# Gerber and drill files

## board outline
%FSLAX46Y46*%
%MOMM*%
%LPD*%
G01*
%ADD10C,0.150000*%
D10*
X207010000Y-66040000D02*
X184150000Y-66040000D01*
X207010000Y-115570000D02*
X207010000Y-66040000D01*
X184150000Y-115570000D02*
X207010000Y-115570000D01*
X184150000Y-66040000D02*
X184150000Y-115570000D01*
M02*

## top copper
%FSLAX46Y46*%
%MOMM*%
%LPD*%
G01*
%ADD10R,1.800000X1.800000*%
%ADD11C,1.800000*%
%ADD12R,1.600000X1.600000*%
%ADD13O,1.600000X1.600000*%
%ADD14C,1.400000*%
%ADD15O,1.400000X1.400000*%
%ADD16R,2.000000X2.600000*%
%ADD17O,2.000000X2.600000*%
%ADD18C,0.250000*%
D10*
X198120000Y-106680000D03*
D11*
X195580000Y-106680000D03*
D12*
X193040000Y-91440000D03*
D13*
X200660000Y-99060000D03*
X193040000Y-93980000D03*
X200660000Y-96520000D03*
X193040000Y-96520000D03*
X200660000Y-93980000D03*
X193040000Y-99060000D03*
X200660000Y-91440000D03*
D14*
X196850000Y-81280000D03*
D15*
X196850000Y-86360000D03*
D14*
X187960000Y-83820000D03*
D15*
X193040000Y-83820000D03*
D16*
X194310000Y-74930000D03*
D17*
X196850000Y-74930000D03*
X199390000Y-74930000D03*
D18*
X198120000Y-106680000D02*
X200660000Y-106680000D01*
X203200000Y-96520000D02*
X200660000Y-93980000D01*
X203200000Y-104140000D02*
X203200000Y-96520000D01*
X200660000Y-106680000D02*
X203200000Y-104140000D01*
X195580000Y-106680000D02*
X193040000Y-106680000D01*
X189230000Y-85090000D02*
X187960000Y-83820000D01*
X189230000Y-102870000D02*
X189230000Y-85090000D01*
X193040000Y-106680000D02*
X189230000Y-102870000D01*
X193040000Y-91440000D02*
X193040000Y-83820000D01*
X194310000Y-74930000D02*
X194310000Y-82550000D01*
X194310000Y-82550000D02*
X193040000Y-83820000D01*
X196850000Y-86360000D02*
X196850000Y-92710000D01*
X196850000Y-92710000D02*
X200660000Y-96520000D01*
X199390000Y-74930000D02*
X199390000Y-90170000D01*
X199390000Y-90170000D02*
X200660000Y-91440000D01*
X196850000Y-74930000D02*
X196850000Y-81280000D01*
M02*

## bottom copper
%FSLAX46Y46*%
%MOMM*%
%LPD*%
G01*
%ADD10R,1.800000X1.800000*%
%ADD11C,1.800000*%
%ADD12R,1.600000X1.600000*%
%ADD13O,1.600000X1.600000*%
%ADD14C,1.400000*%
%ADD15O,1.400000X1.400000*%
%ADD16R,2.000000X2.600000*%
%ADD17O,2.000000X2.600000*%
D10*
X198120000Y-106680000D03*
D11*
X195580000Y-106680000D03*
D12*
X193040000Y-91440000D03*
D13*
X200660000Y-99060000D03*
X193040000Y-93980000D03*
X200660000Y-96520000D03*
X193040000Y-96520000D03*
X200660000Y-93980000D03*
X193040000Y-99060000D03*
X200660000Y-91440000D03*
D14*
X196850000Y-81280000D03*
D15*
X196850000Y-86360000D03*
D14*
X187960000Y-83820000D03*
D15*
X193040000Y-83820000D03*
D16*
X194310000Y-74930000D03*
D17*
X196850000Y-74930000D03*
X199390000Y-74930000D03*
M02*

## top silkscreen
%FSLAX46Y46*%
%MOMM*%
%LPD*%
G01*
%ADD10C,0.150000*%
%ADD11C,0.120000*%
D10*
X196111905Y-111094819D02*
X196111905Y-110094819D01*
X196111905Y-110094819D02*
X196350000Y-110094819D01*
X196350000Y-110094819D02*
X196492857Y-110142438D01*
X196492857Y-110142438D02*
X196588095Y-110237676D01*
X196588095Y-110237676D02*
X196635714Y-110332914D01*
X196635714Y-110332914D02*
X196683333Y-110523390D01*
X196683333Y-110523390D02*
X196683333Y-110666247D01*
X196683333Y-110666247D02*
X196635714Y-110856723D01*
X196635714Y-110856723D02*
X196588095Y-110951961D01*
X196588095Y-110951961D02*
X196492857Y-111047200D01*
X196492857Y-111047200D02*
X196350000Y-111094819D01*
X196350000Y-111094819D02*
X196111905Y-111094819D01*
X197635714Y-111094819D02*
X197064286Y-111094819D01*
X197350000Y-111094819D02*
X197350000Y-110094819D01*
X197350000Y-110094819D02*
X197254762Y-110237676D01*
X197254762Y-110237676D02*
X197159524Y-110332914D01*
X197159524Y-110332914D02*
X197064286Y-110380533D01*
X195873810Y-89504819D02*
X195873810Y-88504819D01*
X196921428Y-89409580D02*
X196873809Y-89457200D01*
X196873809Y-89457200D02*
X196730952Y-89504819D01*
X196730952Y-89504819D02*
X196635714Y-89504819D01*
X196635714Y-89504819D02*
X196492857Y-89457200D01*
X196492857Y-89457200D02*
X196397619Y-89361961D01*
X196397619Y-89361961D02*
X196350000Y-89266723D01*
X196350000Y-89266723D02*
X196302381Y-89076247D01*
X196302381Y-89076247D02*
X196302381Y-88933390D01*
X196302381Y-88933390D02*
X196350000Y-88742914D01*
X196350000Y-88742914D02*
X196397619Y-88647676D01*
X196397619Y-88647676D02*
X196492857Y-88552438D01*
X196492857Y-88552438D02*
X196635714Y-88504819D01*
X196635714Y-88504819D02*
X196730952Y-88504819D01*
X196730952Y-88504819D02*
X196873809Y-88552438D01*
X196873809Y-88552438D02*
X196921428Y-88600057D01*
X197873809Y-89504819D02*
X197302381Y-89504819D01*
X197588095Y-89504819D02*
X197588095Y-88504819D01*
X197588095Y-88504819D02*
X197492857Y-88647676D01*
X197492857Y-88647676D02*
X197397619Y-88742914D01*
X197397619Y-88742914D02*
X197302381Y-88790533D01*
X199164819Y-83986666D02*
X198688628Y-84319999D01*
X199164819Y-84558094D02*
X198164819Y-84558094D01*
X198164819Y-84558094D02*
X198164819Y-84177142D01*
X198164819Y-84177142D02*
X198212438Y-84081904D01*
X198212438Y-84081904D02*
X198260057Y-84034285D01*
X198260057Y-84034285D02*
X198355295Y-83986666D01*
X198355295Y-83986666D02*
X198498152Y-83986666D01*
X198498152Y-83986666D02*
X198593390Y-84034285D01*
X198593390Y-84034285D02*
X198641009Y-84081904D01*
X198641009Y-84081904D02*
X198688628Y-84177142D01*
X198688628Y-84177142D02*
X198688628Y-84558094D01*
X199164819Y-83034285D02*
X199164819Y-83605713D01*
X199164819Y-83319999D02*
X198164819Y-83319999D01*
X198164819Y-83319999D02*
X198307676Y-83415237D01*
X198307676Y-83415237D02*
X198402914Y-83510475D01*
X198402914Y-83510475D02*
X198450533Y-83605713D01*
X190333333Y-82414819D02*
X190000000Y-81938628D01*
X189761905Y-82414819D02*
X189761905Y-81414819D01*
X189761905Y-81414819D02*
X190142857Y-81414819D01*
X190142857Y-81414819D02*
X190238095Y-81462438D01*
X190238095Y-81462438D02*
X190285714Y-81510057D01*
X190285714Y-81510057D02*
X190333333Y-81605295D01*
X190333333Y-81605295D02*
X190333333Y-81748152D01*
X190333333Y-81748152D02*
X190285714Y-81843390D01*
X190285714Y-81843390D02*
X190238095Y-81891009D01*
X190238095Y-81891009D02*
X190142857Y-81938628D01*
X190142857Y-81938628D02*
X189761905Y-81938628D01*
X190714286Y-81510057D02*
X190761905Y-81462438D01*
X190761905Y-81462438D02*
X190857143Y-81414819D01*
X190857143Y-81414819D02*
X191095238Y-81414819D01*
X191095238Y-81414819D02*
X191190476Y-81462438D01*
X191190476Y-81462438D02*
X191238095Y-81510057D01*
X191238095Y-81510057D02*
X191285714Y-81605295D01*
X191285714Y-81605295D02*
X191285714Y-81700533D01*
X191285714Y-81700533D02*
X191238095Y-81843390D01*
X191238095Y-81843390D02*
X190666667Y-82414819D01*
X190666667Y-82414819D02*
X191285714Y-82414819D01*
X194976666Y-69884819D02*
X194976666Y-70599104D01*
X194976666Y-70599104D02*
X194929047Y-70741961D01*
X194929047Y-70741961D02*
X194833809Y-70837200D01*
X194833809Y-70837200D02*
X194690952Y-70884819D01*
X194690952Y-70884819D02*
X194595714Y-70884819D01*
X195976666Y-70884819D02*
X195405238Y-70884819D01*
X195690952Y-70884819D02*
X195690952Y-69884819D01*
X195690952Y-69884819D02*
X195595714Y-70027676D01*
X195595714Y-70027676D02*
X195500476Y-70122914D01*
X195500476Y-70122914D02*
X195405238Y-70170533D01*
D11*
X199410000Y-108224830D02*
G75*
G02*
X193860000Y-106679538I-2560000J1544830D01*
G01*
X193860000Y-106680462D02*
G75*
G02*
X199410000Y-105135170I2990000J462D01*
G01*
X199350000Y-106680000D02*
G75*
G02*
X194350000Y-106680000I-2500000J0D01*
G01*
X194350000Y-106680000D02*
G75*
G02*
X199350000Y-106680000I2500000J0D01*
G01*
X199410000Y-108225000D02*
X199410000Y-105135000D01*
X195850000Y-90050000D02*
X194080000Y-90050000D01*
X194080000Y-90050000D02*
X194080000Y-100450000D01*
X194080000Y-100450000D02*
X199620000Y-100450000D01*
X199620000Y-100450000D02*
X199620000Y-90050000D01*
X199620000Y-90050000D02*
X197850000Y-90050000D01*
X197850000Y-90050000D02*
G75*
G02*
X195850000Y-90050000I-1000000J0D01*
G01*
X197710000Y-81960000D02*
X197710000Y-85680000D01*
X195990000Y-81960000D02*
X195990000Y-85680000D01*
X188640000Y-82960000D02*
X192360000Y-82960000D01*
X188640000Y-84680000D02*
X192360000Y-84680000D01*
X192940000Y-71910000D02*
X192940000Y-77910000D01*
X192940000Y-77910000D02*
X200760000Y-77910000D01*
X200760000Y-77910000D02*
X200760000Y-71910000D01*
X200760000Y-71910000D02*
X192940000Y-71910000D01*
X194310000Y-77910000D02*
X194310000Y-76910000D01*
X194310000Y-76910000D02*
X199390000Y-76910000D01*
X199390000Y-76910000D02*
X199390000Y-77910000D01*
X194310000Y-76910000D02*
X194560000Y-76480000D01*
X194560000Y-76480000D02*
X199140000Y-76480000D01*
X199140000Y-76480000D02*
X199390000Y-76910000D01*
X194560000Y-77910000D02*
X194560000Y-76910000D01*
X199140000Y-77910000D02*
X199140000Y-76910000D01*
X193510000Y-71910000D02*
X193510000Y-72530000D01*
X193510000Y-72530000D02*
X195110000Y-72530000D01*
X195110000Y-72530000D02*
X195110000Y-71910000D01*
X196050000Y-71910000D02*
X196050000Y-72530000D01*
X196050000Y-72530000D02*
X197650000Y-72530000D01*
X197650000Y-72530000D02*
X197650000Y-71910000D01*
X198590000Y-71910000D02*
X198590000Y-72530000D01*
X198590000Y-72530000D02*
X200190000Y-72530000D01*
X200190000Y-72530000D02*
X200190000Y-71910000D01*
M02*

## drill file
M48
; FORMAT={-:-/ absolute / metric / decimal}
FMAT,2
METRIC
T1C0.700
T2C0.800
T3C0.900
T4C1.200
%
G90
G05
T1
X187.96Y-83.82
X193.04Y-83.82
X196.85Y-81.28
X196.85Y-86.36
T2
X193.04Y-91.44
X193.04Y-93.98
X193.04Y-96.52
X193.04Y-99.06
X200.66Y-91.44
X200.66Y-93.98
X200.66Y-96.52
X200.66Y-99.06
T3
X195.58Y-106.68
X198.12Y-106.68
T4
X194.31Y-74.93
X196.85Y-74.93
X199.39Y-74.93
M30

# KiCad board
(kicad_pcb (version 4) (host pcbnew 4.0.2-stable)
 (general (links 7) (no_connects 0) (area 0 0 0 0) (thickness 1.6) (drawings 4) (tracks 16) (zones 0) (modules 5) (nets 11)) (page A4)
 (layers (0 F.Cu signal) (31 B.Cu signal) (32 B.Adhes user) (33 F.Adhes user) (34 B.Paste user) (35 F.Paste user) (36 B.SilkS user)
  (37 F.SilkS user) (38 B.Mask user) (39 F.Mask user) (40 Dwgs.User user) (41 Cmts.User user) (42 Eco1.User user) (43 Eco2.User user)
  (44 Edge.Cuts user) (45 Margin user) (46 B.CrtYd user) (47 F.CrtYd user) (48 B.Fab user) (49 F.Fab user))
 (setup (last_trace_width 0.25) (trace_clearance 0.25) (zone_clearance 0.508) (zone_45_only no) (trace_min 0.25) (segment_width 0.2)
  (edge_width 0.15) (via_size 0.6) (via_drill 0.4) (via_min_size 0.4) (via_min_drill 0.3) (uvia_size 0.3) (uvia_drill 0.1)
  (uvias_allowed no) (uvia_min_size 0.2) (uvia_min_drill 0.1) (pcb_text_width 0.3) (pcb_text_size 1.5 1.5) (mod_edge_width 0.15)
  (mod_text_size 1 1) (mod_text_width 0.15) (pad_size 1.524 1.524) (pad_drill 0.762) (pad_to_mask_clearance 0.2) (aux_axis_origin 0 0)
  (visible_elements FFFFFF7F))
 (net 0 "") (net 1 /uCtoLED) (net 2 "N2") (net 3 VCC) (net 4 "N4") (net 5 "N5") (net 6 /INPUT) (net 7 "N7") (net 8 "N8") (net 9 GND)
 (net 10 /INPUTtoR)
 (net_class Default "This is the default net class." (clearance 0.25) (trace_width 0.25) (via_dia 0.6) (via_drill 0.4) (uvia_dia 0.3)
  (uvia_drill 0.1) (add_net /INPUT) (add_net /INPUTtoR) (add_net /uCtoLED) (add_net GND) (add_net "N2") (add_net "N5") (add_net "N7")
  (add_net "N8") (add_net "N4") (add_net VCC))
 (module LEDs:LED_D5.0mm (layer F.Cu) (at 198.12 106.68 180)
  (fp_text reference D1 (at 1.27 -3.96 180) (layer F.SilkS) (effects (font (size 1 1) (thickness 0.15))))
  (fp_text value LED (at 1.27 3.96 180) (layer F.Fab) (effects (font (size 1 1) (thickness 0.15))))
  (fp_arc (start 1.27 0) (end -1.29 -1.54483) (angle 148.9) (layer F.SilkS) (width 0.12))
  (fp_arc (start 1.27 0) (end -1.29 1.54483) (angle -148.9) (layer F.SilkS) (width 0.12))
  (fp_circle (center 1.27 0) (end 3.77 0) (layer F.SilkS) (width 0.12))
  (fp_line (start -1.29 -1.545) (end -1.29 1.545) (layer F.SilkS) (width 0.12))
  (pad 1 thru_hole rect (at 0 0 180) (size 1.8 1.8) (drill 0.9) (layers *.Cu *.Mask) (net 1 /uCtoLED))
  (pad 2 thru_hole circle (at 2.54 0 180) (size 1.8 1.8) (drill 0.9) (layers *.Cu *.Mask) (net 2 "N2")))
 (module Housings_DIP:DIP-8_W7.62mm (layer F.Cu) (at 193.04 91.44)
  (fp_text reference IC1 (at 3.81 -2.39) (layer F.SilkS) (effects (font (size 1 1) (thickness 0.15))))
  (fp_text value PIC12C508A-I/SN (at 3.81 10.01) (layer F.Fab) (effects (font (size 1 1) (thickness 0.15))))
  (fp_line (start 2.81 -1.39) (end 1.04 -1.39) (layer F.SilkS) (width 0.12))
  (fp_line (start 1.04 -1.39) (end 1.04 9.01) (layer F.SilkS) (width 0.12))
  (fp_line (start 1.04 9.01) (end 6.58 9.01) (layer F.SilkS) (width 0.12))
  (fp_line (start 6.58 9.01) (end 6.58 -1.39) (layer F.SilkS) (width 0.12))
  (fp_line (start 6.58 -1.39) (end 4.81 -1.39) (layer F.SilkS) (width 0.12))
  (fp_arc (start 3.81 -1.39) (end 2.81 -1.39) (angle -180) (layer F.SilkS) (width 0.12))
  (pad 1 thru_hole rect (at 0 0) (size 1.6 1.6) (drill 0.8) (layers *.Cu *.Mask) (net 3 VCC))
  (pad 5 thru_hole oval (at 7.62 7.62) (size 1.6 1.6) (drill 0.8) (layers *.Cu *.Mask) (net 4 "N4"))
  (pad 2 thru_hole oval (at 0 2.54) (size 1.6 1.6) (drill 0.8) (layers *.Cu *.Mask) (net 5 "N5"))
  (pad 6 thru_hole oval (at 7.62 5.08) (size 1.6 1.6) (drill 0.8) (layers *.Cu *.Mask) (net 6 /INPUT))
  (pad 3 thru_hole oval (at 0 5.08) (size 1.6 1.6) (drill 0.8) (layers *.Cu *.Mask) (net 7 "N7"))
  (pad 7 thru_hole oval (at 7.62 2.54) (size 1.6 1.6) (drill 0.8) (layers *.Cu *.Mask) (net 1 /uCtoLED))
  (pad 4 thru_hole oval (at 0 7.62) (size 1.6 1.6) (drill 0.8) (layers *.Cu *.Mask) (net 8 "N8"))
  (pad 8 thru_hole oval (at 7.62 0) (size 1.6 1.6) (drill 0.8) (layers *.Cu *.Mask) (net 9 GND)))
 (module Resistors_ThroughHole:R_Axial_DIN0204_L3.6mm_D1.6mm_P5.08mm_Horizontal (layer F.Cu) (at 196.85 81.28 270)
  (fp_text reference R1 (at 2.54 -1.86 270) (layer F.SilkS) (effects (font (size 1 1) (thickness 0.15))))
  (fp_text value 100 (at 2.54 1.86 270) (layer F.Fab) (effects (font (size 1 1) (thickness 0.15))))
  (fp_line (start 0.68 -0.86) (end 4.4 -0.86) (layer F.SilkS) (width 0.12))
  (fp_line (start 0.68 0.86) (end 4.4 0.86) (layer F.SilkS) (width 0.12))
  (pad 1 thru_hole circle (at 0 0 270) (size 1.4 1.4) (drill 0.7) (layers *.Cu *.Mask) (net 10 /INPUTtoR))
  (pad 2 thru_hole oval (at 5.08 0 270) (size 1.4 1.4) (drill 0.7) (layers *.Cu *.Mask) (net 6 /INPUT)))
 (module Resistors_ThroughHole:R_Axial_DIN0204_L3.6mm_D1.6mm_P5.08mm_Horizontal (layer F.Cu) (at 187.96 83.82)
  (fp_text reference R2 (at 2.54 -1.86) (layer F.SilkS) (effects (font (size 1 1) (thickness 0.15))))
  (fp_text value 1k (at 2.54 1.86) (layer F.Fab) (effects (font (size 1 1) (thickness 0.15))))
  (fp_line (start 0.68 -0.86) (end 4.4 -0.86) (layer F.SilkS) (width 0.12))
  (fp_line (start 0.68 0.86) (end 4.4 0.86) (layer F.SilkS) (width 0.12))
  (pad 1 thru_hole circle (at 0 0) (size 1.4 1.4) (drill 0.7) (layers *.Cu *.Mask) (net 2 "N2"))
  (pad 2 thru_hole oval (at 5.08 0) (size 1.4 1.4) (drill 0.7) (layers *.Cu *.Mask) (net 3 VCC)))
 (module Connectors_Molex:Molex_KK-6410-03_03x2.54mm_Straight (layer F.Cu) (at 194.31 74.93)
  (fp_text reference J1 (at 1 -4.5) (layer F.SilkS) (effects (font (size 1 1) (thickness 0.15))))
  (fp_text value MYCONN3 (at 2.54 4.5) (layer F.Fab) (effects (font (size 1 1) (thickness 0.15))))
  (fp_line (start -1.37 -3.02) (end -1.37 2.98) (layer F.SilkS) (width 0.12))
  (fp_line (start -1.37 2.98) (end 6.45 2.98) (layer F.SilkS) (width 0.12))
  (fp_line (start 6.45 2.98) (end 6.45 -3.02) (layer F.SilkS) (width 0.12))
  (fp_line (start 6.45 -3.02) (end -1.37 -3.02) (layer F.SilkS) (width 0.12))
  (fp_line (start 0 2.98) (end 0 1.98) (layer F.SilkS) (width 0.12))
  (fp_line (start 0 1.98) (end 5.08 1.98) (layer F.SilkS) (width 0.12))
  (fp_line (start 5.08 1.98) (end 5.08 2.98) (layer F.SilkS) (width 0.12))
  (fp_line (start 0 1.98) (end 0.25 1.55) (layer F.SilkS) (width 0.12))
  (fp_line (start 0.25 1.55) (end 4.83 1.55) (layer F.SilkS) (width 0.12))
  (fp_line (start 4.83 1.55) (end 5.08 1.98) (layer F.SilkS) (width 0.12))
  (fp_line (start 0.25 2.98) (end 0.25 1.98) (layer F.SilkS) (width 0.12))
  (fp_line (start 4.83 2.98) (end 4.83 1.98) (layer F.SilkS) (width 0.12))
  (fp_line (start -0.8 -3.02) (end -0.8 -2.4) (layer F.SilkS) (width 0.12))
  (fp_line (start -0.8 -2.4) (end 0.8 -2.4) (layer F.SilkS) (width 0.12))
  (fp_line (start 0.8 -2.4) (end 0.8 -3.02) (layer F.SilkS) (width 0.12))
  (fp_line (start 1.74 -3.02) (end 1.74 -2.4) (layer F.SilkS) (width 0.12))
  (fp_line (start 1.74 -2.4) (end 3.34 -2.4) (layer F.SilkS) (width 0.12))
  (fp_line (start 3.34 -2.4) (end 3.34 -3.02) (layer F.SilkS) (width 0.12))
  (fp_line (start 4.28 -3.02) (end 4.28 -2.4) (layer F.SilkS) (width 0.12))
  (fp_line (start 4.28 -2.4) (end 5.88 -2.4) (layer F.SilkS) (width 0.12))
  (fp_line (start 5.88 -2.4) (end 5.88 -3.02) (layer F.SilkS) (width 0.12))
  (pad 1 thru_hole rect (at 0 0) (size 2 2.6) (drill 1.2) (layers *.Cu *.Mask) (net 3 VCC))
  (pad 2 thru_hole oval (at 2.54 0) (size 2 2.6) (drill 1.2) (layers *.Cu *.Mask) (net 10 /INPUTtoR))
  (pad 3 thru_hole oval (at 5.08 0) (size 2 2.6) (drill 1.2) (layers *.Cu *.Mask) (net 9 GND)))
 (gr_line (start 207.01 66.04) (end 184.15 66.04) (angle 90) (layer Edge.Cuts) (width 0.15))
 (gr_line (start 207.01 115.57) (end 207.01 66.04) (angle 90) (layer Edge.Cuts) (width 0.15))
 (gr_line (start 184.15 115.57) (end 207.01 115.57) (angle 90) (layer Edge.Cuts) (width 0.15))
 (gr_line (start 184.15 66.04) (end 184.15 115.57) (angle 90) (layer Edge.Cuts) (width 0.15))
 (segment (start 198.12 106.68) (end 200.66 106.68) (width 0.25) (layer F.Cu) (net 1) (status 400000))
 (segment (start 203.2 96.52) (end 200.66 93.98) (width 0.25) (layer F.Cu) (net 1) (status 800000))
 (segment (start 203.2 104.14) (end 203.2 96.52) (width 0.25) (layer F.Cu) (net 1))
 (segment (start 200.66 106.68) (end 203.2 104.14) (width 0.25) (layer F.Cu) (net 1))
 (segment (start 195.58 106.68) (end 193.04 106.68) (width 0.25) (layer F.Cu) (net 2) (status 400000))
 (segment (start 189.23 85.09) (end 187.96 83.82) (width 0.25) (layer F.Cu) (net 2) (status 800000))
 (segment (start 189.23 102.87) (end 189.23 85.09) (width 0.25) (layer F.Cu) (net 2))
 (segment (start 193.04 106.68) (end 189.23 102.87) (width 0.25) (layer F.Cu) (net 2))
 (segment (start 193.04 91.44) (end 193.04 83.82) (width 0.25) (layer F.Cu) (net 3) (status C00000))
 (segment (start 194.31 74.93) (end 194.31 82.55) (width 0.25) (layer F.Cu) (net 3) (status 400000))
 (segment (start 194.31 82.55) (end 193.04 83.82) (width 0.25) (layer F.Cu) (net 3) (status 800000))
 (segment (start 196.85 86.36) (end 196.85 92.71) (width 0.25) (layer F.Cu) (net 6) (status 400000))
 (segment (start 196.85 92.71) (end 200.66 96.52) (width 0.25) (layer F.Cu) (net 6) (status 800000))
 (segment (start 199.39 74.93) (end 199.39 90.17) (width 0.25) (layer F.Cu) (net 9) (status 400000))
 (segment (start 199.39 90.17) (end 200.66 91.44) (width 0.25) (layer F.Cu) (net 9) (status 800000))
 (segment (start 196.85 74.93) (end 196.85 81.28) (width 0.25) (layer F.Cu) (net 10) (status C00000)))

